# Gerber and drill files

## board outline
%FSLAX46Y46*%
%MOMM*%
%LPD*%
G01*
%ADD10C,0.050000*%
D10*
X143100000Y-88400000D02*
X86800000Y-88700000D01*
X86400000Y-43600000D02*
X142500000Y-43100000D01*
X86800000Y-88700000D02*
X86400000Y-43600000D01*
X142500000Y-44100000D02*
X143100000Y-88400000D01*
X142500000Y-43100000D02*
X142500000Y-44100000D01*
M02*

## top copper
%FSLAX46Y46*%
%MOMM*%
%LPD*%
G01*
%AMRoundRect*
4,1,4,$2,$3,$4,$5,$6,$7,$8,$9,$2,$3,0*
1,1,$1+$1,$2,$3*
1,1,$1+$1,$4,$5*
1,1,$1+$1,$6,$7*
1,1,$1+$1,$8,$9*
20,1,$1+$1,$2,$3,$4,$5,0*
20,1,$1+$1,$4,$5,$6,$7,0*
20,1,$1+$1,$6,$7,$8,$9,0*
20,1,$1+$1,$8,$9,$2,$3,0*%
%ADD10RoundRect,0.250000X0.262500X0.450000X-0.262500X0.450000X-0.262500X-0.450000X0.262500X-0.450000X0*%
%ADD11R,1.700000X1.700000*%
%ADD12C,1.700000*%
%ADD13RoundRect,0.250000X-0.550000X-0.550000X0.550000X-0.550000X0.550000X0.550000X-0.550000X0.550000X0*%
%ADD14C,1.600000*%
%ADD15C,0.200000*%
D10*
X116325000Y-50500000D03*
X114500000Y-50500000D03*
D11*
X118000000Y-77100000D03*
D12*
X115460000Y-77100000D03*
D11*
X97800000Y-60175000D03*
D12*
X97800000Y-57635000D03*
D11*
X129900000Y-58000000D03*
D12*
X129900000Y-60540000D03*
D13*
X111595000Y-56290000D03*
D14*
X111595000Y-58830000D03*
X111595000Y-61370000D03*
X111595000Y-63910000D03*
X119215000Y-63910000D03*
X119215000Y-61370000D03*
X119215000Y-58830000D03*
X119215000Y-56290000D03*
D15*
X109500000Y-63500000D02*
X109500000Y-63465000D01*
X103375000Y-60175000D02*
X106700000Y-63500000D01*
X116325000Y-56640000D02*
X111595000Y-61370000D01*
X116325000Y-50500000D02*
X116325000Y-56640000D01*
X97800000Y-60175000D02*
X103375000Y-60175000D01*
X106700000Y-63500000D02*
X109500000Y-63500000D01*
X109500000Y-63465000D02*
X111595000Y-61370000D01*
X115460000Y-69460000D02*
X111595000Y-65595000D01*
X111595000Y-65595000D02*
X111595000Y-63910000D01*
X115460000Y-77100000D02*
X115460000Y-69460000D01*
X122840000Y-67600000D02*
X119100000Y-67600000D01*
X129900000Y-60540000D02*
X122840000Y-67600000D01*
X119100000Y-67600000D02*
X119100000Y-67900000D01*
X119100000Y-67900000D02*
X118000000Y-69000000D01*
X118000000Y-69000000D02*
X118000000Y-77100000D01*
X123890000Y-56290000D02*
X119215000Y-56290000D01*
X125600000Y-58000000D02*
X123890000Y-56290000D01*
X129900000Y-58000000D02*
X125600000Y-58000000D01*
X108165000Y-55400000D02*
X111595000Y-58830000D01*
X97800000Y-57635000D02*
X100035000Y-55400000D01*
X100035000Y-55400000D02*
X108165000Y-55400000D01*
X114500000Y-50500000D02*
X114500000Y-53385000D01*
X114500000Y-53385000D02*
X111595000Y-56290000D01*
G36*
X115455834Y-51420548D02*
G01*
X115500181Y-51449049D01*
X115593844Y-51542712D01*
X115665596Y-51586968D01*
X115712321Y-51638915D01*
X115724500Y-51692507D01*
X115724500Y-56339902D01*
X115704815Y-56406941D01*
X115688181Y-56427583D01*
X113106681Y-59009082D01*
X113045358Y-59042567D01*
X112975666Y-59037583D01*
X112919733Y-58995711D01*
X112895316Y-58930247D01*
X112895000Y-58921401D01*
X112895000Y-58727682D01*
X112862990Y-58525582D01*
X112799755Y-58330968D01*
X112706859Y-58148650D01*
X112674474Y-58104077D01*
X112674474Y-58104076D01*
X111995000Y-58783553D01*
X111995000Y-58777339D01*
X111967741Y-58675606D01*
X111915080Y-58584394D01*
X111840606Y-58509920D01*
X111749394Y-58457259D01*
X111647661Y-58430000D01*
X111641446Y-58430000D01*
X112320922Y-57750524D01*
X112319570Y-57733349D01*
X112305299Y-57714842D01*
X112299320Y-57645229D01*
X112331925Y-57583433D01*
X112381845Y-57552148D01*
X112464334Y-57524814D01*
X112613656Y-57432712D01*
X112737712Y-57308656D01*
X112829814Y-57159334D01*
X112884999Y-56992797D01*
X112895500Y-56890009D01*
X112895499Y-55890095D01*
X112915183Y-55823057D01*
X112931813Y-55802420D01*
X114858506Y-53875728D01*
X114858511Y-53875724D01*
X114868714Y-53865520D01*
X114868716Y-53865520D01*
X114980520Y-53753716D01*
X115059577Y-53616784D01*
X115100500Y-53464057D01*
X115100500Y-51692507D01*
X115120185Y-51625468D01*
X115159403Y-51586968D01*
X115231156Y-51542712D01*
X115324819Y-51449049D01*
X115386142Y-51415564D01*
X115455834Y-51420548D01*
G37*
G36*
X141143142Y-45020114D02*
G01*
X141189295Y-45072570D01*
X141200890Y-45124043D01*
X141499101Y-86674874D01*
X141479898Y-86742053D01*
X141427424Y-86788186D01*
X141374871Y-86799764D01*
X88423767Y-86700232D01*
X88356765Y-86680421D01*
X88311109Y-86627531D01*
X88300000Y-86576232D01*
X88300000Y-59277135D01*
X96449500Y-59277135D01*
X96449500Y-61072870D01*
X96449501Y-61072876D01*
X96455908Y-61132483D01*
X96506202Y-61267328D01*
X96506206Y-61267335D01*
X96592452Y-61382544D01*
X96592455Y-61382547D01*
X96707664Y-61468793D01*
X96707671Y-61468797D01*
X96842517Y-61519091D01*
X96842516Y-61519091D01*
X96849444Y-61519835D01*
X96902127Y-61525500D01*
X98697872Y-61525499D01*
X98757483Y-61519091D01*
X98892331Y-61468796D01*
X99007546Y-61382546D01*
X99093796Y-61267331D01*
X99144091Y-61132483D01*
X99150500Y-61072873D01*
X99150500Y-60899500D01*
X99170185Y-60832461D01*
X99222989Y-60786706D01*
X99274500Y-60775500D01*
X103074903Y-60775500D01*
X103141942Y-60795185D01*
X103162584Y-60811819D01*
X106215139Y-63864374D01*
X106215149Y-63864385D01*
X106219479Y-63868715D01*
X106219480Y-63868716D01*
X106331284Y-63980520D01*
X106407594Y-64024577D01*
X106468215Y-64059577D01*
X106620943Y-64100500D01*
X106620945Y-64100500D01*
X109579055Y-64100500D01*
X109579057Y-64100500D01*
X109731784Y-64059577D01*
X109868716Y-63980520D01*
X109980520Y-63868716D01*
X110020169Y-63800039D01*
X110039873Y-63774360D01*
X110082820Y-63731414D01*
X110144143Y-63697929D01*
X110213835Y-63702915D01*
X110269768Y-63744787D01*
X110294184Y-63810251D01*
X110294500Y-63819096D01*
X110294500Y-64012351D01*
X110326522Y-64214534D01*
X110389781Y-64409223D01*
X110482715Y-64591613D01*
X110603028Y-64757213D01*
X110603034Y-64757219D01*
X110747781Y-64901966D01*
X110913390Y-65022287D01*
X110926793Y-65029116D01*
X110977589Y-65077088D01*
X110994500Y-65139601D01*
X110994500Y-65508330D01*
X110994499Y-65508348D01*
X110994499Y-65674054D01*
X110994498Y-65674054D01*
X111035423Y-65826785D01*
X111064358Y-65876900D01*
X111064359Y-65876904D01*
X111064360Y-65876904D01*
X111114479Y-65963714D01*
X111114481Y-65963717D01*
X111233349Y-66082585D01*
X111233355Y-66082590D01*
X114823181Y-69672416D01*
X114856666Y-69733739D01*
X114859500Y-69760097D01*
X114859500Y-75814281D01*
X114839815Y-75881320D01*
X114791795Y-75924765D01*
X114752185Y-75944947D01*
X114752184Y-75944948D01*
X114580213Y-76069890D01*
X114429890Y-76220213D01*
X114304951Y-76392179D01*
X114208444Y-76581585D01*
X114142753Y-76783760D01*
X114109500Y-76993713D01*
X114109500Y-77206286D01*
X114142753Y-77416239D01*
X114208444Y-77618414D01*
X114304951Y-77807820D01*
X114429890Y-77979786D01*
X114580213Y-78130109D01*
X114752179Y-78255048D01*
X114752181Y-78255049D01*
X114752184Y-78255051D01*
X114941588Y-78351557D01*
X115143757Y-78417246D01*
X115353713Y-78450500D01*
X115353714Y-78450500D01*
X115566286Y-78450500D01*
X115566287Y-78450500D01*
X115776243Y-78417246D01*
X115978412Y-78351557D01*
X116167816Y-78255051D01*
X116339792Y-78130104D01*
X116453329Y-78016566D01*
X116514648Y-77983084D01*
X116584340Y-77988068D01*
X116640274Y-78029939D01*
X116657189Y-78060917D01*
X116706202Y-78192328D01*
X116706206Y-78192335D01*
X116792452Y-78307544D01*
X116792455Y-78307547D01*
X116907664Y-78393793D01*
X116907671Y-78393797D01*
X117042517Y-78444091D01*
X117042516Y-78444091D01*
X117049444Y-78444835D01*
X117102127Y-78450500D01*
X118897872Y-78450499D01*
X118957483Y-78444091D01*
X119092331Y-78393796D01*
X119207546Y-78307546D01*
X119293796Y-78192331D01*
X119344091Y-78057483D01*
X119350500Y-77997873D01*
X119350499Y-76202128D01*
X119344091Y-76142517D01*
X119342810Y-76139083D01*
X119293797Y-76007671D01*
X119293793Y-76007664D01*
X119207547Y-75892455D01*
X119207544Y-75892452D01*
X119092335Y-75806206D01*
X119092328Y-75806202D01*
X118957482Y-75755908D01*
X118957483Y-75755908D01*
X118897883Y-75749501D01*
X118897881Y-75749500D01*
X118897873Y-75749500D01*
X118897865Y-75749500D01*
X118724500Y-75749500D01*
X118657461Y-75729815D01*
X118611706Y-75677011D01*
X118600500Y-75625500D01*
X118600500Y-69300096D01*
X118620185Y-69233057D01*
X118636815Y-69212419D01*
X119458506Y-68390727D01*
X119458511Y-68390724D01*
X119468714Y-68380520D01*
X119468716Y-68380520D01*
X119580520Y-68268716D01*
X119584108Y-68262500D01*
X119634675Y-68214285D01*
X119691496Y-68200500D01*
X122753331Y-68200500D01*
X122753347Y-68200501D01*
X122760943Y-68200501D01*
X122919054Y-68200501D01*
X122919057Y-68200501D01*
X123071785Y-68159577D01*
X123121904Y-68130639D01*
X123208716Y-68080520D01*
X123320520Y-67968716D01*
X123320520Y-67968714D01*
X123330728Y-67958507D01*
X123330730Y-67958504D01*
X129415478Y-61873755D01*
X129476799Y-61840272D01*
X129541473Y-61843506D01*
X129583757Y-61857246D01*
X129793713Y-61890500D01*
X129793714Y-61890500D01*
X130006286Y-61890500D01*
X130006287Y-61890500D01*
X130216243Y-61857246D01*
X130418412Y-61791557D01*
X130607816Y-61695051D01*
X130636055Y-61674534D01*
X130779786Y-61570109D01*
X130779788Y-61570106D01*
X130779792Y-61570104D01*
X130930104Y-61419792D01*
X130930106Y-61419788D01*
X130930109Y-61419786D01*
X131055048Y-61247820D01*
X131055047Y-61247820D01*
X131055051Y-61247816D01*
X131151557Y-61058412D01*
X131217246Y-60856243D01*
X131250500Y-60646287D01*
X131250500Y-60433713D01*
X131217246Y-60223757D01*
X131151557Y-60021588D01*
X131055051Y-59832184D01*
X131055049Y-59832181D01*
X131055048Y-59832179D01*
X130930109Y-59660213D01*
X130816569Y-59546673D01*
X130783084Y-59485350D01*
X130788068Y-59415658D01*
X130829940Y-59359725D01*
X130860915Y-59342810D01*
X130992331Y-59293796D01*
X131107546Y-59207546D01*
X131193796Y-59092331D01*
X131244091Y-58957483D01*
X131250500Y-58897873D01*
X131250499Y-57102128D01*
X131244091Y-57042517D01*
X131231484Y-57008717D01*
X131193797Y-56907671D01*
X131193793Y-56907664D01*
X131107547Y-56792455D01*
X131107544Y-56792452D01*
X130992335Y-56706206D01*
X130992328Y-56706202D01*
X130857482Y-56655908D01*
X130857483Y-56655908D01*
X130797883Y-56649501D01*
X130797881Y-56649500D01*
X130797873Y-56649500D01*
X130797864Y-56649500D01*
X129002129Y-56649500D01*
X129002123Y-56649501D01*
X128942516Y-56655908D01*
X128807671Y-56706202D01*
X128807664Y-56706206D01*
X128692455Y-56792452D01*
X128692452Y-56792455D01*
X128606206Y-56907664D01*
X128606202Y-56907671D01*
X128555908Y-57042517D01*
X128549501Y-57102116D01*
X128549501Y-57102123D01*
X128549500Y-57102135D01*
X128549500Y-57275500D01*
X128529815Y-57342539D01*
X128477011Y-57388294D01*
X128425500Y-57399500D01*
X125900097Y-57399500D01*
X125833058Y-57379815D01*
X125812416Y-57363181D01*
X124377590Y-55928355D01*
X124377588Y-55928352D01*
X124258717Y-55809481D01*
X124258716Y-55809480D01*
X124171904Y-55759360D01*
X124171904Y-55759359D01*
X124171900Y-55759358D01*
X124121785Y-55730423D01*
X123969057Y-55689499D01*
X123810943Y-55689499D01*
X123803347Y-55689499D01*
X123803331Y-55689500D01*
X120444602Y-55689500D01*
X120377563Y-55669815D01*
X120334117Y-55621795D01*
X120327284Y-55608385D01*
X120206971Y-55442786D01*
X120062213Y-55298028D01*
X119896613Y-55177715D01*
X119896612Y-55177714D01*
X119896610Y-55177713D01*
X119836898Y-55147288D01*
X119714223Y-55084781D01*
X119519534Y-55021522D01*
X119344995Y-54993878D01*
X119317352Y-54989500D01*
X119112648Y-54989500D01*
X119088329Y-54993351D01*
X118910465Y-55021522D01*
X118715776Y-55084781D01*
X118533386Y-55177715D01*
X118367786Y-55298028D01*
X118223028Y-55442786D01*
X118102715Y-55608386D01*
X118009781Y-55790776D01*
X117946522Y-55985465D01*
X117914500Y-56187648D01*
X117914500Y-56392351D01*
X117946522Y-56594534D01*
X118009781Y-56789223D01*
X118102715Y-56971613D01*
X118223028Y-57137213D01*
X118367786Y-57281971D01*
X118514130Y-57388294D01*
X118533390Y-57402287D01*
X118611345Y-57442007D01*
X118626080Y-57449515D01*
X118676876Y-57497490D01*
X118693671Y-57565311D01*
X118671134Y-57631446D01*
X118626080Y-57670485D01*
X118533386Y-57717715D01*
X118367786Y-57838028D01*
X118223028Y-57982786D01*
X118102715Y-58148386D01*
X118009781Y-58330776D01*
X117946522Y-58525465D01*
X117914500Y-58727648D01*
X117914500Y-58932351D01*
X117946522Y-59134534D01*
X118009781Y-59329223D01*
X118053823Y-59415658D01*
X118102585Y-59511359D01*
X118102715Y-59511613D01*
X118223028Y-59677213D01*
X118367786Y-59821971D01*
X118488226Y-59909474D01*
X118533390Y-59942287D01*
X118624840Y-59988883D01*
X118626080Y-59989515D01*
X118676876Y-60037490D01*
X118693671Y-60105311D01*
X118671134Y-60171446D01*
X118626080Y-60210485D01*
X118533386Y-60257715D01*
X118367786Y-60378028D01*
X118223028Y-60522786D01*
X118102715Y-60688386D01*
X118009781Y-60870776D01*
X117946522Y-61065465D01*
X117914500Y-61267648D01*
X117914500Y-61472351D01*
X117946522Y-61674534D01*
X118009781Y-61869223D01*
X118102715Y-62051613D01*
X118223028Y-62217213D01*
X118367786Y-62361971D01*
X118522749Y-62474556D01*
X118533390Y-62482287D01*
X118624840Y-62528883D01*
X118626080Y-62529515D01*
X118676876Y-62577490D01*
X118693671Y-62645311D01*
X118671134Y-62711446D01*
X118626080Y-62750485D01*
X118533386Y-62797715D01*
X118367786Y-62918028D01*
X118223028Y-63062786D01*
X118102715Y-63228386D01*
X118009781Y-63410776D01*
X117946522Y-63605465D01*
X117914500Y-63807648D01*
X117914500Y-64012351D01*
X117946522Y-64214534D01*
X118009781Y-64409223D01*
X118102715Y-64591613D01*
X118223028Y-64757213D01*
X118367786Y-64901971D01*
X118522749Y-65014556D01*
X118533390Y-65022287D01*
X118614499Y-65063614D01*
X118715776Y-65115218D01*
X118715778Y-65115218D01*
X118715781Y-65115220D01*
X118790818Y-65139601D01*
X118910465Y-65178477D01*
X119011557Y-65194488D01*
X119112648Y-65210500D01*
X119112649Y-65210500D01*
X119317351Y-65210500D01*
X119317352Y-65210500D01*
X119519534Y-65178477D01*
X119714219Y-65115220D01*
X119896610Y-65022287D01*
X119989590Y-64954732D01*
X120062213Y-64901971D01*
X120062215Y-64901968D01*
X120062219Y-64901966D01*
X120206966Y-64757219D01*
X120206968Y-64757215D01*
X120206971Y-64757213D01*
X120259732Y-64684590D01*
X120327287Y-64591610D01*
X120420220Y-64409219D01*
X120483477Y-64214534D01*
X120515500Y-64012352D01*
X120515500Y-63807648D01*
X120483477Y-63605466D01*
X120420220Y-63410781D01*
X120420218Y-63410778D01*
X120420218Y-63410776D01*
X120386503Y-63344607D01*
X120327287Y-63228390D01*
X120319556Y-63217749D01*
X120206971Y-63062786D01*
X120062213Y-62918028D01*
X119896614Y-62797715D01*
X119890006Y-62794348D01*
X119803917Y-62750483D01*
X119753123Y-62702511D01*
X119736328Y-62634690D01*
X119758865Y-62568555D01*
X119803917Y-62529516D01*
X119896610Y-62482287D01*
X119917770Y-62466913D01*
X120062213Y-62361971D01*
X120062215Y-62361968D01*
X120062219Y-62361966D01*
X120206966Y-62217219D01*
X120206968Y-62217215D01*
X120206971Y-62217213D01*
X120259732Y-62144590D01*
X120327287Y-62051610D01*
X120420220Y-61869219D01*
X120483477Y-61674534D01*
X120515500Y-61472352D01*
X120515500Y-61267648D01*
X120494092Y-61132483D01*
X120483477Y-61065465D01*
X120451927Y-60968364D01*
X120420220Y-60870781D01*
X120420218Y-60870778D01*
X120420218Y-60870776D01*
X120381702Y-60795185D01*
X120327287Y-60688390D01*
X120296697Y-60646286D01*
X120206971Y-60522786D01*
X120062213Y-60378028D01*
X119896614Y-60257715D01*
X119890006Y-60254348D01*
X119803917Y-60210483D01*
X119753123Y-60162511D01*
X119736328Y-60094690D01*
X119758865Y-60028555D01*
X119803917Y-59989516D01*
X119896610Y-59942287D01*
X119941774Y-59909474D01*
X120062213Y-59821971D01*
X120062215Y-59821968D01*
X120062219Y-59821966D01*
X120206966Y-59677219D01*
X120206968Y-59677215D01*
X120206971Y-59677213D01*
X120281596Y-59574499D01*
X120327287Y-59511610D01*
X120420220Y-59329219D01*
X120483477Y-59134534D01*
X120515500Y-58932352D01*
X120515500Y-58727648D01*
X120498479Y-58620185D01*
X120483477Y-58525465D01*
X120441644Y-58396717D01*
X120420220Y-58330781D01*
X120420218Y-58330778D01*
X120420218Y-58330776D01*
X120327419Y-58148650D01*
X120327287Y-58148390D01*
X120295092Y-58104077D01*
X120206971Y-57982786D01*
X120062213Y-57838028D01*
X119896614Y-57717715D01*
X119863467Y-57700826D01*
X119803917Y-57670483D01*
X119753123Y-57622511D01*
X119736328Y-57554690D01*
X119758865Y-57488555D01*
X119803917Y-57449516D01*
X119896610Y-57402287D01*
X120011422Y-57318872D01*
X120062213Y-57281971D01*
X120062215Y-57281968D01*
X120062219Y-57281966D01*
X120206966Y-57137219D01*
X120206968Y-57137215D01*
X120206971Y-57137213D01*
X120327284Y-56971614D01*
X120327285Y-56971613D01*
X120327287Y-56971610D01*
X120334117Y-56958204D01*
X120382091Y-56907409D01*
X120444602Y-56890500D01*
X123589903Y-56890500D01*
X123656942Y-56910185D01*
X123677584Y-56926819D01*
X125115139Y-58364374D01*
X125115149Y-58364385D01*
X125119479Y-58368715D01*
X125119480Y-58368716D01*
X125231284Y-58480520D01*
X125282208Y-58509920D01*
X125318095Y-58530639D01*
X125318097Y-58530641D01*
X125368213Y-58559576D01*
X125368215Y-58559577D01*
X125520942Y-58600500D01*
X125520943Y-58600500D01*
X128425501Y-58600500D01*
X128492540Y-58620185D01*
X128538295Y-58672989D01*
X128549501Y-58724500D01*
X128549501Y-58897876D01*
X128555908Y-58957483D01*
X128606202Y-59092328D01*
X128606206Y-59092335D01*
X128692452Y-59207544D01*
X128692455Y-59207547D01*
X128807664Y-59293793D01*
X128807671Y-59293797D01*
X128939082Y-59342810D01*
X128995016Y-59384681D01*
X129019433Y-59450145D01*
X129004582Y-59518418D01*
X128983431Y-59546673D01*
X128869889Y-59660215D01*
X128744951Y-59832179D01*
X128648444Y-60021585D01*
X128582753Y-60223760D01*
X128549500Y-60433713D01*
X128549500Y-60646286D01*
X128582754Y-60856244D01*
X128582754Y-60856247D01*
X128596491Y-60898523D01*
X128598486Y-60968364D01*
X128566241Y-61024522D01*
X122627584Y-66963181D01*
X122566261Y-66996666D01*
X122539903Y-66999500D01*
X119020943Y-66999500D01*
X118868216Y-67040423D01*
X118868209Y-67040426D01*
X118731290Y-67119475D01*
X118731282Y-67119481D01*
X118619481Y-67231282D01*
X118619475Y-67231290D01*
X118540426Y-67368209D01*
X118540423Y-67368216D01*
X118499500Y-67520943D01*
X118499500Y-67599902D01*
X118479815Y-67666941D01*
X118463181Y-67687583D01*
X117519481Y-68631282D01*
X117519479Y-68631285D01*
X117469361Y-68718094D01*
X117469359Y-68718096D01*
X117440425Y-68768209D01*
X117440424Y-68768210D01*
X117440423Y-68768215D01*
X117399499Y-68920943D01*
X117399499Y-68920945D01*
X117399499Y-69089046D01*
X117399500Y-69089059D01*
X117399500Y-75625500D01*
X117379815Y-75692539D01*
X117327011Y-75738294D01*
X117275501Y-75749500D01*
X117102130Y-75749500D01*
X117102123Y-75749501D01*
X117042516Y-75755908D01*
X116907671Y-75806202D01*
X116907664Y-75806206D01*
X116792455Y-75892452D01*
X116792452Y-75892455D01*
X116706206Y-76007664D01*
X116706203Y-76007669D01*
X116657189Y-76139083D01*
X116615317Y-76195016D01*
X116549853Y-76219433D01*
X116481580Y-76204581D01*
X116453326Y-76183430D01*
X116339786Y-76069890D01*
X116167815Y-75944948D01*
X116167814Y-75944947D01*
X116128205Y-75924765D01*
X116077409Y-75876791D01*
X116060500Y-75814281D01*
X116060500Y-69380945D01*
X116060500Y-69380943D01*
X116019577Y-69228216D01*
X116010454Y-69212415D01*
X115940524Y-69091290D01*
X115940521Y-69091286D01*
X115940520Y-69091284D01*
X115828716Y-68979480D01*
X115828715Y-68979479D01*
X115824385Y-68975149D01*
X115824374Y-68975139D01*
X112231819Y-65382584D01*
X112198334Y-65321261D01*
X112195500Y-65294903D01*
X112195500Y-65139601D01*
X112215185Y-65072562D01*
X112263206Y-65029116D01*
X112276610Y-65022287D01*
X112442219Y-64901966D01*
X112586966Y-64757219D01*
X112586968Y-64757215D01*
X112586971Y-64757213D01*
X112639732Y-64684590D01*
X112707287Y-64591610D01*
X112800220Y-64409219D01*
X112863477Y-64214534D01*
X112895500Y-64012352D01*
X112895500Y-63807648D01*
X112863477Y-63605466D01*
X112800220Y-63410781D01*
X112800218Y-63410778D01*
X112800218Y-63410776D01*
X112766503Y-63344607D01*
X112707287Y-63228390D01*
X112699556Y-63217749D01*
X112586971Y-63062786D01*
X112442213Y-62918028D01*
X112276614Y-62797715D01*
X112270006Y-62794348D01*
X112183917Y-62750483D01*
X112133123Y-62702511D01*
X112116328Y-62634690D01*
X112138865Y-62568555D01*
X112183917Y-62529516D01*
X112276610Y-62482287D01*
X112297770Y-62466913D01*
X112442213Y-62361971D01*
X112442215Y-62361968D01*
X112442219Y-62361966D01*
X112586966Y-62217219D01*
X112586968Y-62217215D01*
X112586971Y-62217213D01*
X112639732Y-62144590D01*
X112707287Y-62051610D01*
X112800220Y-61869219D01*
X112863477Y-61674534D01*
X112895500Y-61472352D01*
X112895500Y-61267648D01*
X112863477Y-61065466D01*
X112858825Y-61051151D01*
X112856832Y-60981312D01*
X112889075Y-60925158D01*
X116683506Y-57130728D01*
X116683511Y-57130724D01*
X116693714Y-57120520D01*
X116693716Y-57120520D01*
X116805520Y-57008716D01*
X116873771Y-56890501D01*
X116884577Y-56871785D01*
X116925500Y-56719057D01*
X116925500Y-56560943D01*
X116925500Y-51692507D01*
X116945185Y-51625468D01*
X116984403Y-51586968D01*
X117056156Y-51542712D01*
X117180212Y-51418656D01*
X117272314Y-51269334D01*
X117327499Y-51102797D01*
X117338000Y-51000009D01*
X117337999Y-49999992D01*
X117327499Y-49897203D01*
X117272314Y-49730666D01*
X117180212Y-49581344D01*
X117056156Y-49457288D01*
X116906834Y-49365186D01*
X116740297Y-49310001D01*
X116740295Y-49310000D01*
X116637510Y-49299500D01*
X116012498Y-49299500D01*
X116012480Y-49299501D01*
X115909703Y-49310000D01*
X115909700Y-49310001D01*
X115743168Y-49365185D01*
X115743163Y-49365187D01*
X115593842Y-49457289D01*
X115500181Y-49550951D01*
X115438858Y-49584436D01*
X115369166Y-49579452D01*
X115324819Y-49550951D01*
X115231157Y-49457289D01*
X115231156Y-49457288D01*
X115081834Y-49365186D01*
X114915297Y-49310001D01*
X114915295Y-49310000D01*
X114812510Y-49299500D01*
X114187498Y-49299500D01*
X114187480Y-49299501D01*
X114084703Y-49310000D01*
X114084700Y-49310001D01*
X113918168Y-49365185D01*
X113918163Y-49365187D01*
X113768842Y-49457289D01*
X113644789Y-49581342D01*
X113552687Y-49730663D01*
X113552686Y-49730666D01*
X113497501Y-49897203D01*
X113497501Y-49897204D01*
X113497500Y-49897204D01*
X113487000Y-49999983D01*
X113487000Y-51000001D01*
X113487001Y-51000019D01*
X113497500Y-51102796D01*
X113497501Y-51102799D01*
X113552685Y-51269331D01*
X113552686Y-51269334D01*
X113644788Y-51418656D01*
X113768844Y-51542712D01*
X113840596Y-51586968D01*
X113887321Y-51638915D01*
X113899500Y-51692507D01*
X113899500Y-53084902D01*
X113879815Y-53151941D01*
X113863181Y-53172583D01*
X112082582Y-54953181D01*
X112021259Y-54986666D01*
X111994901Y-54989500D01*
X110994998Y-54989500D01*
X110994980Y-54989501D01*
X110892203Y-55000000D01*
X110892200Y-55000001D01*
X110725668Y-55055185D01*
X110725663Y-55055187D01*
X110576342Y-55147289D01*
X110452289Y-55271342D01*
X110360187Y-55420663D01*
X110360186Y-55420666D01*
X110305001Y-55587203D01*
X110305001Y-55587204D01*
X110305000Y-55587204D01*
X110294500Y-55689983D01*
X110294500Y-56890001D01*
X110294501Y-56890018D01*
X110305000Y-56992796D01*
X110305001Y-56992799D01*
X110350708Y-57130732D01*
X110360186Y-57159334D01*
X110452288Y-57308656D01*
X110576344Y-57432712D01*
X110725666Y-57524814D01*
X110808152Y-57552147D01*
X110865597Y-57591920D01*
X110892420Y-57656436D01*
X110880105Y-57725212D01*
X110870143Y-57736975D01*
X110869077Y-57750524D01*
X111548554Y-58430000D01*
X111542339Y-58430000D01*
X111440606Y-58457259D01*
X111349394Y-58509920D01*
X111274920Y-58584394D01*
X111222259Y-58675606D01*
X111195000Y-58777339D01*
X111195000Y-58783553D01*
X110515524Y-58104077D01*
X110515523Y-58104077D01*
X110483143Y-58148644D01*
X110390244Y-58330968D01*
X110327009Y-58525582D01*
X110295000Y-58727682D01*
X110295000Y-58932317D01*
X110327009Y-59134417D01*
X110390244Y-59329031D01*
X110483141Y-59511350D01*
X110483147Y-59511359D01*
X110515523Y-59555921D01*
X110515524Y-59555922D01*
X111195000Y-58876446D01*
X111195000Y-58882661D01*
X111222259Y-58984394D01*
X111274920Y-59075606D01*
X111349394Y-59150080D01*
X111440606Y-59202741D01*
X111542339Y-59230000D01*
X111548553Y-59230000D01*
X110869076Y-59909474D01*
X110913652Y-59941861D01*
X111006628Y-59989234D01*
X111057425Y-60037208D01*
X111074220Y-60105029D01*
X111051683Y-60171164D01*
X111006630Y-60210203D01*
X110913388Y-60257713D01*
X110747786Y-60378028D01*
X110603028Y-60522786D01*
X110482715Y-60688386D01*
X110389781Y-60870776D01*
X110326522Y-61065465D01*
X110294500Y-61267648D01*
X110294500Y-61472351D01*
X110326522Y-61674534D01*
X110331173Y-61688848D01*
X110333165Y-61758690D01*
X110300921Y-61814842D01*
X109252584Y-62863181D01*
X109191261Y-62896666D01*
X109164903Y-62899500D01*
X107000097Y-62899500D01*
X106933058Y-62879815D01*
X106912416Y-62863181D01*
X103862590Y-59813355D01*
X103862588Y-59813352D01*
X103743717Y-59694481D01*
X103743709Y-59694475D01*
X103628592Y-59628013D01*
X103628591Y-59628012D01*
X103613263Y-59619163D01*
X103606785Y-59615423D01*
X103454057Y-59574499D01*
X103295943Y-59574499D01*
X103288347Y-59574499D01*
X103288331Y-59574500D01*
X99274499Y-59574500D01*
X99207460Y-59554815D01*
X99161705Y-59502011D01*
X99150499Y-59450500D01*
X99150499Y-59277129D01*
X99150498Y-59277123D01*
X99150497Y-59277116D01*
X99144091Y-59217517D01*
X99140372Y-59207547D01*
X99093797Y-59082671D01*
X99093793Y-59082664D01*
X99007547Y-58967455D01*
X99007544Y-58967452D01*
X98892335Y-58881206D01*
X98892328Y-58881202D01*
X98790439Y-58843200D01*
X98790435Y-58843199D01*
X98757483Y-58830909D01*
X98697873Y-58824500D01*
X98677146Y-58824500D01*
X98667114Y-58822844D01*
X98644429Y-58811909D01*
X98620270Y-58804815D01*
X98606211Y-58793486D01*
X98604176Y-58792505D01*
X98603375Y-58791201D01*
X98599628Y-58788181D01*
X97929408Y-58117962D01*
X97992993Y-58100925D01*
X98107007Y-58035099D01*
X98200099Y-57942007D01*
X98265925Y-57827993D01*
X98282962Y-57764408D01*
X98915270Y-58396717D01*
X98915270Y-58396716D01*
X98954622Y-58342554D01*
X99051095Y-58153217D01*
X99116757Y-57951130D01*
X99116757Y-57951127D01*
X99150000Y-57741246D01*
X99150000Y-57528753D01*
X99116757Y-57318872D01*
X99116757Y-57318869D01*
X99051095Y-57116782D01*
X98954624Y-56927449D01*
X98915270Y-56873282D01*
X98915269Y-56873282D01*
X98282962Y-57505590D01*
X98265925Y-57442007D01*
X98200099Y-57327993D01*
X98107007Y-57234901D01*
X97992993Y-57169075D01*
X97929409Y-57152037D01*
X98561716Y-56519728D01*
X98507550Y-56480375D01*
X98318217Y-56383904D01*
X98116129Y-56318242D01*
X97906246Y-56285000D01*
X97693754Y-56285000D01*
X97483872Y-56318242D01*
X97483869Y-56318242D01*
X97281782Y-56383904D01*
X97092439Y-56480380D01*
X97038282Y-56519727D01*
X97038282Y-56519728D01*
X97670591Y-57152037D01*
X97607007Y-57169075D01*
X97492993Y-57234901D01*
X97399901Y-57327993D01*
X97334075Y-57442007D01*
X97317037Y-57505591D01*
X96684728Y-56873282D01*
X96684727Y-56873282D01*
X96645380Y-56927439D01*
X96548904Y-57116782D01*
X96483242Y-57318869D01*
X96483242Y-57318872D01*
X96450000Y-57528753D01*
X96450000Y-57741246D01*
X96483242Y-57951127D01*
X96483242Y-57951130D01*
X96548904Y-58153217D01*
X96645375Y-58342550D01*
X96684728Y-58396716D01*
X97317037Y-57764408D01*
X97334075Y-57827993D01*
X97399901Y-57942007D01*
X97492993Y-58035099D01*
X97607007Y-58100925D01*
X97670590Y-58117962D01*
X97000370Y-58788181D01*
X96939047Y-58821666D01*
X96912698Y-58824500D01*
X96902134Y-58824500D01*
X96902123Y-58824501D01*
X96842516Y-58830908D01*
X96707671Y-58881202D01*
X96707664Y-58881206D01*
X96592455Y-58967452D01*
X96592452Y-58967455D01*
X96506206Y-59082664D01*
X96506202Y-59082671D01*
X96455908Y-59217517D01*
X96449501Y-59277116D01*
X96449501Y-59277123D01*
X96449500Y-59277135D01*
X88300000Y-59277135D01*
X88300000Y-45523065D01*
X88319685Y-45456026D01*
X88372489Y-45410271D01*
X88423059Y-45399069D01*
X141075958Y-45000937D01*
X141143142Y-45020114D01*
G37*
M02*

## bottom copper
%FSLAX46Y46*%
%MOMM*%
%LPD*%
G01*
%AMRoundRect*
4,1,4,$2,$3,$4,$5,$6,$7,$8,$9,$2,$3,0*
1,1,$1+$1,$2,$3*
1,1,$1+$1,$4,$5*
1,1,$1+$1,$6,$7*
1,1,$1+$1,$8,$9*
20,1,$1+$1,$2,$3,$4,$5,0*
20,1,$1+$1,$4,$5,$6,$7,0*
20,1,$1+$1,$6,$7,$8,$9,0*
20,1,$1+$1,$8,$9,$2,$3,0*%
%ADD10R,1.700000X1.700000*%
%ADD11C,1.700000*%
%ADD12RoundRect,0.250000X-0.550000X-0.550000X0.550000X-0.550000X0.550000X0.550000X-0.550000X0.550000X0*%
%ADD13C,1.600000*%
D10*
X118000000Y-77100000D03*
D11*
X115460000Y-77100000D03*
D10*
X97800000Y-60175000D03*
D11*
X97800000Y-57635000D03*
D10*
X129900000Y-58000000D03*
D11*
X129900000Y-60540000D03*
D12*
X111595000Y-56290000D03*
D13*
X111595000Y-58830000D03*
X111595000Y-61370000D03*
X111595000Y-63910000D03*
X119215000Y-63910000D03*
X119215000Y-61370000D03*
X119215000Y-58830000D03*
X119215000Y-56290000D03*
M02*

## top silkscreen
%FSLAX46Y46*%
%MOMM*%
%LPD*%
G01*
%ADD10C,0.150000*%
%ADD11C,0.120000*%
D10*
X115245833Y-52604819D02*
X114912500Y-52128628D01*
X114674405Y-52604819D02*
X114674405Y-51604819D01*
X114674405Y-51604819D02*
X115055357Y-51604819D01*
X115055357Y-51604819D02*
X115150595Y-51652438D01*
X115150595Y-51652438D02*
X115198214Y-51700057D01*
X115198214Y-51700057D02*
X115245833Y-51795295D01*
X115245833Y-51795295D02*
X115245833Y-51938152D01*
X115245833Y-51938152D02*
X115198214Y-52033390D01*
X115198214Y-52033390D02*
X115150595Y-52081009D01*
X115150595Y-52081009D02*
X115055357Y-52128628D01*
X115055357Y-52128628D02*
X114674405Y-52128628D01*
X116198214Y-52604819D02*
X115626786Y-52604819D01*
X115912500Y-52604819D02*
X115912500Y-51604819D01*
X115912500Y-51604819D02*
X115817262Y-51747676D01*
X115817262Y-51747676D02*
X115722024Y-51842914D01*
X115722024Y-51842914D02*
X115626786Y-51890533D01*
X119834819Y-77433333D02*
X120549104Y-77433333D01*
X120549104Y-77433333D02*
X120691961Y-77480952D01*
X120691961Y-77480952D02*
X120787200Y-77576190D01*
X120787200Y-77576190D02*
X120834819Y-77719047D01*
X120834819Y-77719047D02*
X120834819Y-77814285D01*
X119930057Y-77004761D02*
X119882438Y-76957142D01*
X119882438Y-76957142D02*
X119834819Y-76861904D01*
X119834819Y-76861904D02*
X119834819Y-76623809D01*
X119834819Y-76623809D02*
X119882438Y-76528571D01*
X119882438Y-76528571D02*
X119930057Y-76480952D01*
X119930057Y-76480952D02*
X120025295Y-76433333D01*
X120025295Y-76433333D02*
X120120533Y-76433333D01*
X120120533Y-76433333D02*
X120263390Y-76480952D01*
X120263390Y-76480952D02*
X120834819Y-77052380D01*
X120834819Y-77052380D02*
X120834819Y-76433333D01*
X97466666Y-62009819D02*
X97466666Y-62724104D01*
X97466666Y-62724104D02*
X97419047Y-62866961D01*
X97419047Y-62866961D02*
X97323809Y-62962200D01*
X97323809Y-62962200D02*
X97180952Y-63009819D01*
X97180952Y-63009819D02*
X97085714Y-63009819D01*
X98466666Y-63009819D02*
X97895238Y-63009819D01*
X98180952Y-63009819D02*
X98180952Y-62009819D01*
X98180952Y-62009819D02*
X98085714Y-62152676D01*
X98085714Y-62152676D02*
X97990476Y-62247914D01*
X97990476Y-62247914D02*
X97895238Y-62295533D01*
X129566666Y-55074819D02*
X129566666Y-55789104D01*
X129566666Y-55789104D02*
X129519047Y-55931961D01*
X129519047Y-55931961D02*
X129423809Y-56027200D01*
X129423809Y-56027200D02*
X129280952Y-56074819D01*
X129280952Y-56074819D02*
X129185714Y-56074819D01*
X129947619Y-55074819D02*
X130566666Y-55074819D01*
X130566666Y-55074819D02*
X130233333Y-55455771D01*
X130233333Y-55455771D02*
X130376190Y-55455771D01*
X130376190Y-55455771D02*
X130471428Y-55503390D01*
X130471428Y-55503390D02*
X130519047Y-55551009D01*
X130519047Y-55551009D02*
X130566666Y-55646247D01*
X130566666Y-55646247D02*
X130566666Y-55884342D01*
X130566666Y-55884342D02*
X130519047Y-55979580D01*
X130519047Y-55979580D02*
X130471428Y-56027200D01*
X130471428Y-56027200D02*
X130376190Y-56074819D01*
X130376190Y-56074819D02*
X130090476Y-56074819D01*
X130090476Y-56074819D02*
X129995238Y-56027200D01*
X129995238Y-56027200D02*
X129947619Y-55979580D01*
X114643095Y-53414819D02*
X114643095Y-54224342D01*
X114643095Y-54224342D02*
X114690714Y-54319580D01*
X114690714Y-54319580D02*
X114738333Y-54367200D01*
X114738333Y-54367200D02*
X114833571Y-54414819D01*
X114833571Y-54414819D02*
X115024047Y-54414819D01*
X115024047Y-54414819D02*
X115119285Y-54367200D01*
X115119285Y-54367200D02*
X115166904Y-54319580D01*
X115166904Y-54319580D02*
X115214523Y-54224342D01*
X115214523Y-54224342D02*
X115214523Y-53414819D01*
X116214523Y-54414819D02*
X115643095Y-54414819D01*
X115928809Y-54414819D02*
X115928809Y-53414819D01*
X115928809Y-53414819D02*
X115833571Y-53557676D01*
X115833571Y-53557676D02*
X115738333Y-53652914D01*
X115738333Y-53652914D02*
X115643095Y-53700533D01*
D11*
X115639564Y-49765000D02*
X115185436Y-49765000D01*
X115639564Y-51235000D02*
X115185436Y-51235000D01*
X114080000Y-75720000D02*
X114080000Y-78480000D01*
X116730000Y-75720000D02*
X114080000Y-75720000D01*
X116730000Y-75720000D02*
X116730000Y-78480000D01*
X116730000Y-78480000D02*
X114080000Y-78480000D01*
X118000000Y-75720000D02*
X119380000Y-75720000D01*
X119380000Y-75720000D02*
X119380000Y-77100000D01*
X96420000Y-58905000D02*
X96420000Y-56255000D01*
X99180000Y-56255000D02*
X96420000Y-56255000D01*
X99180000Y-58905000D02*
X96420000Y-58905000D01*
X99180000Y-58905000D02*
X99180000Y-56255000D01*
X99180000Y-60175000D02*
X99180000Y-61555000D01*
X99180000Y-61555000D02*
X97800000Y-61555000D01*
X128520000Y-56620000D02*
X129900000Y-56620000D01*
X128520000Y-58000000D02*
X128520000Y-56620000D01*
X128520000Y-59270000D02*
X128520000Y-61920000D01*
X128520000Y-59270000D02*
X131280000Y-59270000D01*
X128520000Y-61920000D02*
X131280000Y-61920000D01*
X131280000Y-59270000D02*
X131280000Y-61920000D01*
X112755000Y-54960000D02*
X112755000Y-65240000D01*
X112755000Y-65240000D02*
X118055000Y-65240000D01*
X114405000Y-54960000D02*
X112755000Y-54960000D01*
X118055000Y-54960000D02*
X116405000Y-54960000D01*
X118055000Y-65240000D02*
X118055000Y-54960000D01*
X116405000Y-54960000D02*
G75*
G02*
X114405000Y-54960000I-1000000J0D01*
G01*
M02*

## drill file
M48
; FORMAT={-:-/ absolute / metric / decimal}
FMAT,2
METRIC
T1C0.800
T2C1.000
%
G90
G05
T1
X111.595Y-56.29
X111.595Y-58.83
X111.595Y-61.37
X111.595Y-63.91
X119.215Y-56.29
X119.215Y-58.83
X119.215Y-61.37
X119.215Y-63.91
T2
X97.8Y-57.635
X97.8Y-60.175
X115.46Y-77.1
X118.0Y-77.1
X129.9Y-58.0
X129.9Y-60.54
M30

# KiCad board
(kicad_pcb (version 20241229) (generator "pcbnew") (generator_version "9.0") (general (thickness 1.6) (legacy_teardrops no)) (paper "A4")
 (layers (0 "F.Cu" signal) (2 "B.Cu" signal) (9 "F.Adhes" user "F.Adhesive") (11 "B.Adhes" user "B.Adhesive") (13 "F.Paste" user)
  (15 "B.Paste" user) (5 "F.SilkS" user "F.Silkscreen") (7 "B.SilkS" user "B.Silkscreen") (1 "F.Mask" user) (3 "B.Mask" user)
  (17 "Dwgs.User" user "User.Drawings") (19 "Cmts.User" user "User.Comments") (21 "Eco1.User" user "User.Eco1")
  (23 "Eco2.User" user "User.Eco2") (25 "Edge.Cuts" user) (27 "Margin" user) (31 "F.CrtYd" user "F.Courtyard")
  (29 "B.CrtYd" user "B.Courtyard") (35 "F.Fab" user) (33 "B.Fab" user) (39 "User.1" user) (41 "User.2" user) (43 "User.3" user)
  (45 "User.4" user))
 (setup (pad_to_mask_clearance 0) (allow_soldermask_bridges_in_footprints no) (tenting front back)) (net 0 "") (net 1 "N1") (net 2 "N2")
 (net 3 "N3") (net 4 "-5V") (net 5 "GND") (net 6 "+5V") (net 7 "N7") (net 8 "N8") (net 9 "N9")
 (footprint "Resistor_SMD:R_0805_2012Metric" (layer "F.Cu") (at 115.4125 50.5 180)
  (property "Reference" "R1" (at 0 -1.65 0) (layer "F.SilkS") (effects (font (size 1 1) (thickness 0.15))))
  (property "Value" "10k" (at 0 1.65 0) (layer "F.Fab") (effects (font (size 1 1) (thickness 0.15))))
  (fp_line (start -0.227064 0.735) (end 0.227064 0.735) (stroke (width 0.12) (type solid)) (layer "F.SilkS"))
  (fp_line (start -0.227064 -0.735) (end 0.227064 -0.735) (stroke (width 0.12) (type solid)) (layer "F.SilkS"))
  (pad "1" smd roundrect (at -0.9125 0 180) (size 1.025 1.4) (layers "F.Cu" "F.Mask" "F.Paste") (roundrect_rratio 0.243902) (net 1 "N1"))
  (pad "2" smd roundrect (at 0.9125 0 180) (size 1.025 1.4) (layers "F.Cu" "F.Mask" "F.Paste") (roundrect_rratio 0.243902) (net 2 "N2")))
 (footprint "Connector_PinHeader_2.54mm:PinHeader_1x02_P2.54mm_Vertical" (layer "F.Cu") (at 118 77.1 -90)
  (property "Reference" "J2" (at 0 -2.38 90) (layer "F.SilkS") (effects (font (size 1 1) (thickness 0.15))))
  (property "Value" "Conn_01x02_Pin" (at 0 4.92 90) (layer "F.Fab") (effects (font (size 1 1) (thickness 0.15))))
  (fp_line (start -1.38 3.92) (end 1.38 3.92) (stroke (width 0.12) (type solid)) (layer "F.SilkS"))
  (fp_line (start -1.38 1.27) (end -1.38 3.92) (stroke (width 0.12) (type solid)) (layer "F.SilkS"))
  (fp_line (start -1.38 1.27) (end 1.38 1.27) (stroke (width 0.12) (type solid)) (layer "F.SilkS"))
  (fp_line (start 1.38 1.27) (end 1.38 3.92) (stroke (width 0.12) (type solid)) (layer "F.SilkS"))
  (fp_line (start -1.38 0) (end -1.38 -1.38) (stroke (width 0.12) (type solid)) (layer "F.SilkS"))
  (fp_line (start -1.38 -1.38) (end 0 -1.38) (stroke (width 0.12) (type solid)) (layer "F.SilkS"))
  (pad "1" thru_hole rect (at 0 0 270) (size 1.7 1.7) (drill 1) (layers "*.Cu" "*.Mask") (remove_unused_layers no) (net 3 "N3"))
  (pad "2" thru_hole circle (at 0 2.54 270) (size 1.7 1.7) (drill 1) (layers "*.Cu" "*.Mask") (remove_unused_layers no) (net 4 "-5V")))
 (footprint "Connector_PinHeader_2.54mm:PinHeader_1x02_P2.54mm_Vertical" (layer "F.Cu") (at 97.8 60.175 180)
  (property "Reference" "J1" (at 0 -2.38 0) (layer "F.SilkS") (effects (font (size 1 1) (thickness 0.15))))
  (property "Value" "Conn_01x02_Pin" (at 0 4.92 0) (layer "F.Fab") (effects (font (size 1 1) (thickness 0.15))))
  (fp_line (start 1.38 1.27) (end 1.38 3.92) (stroke (width 0.12) (type solid)) (layer "F.SilkS"))
  (fp_line (start -1.38 3.92) (end 1.38 3.92) (stroke (width 0.12) (type solid)) (layer "F.SilkS"))
  (fp_line (start -1.38 1.27) (end 1.38 1.27) (stroke (width 0.12) (type solid)) (layer "F.SilkS"))
  (fp_line (start -1.38 1.27) (end -1.38 3.92) (stroke (width 0.12) (type solid)) (layer "F.SilkS"))
  (fp_line (start -1.38 0) (end -1.38 -1.38) (stroke (width 0.12) (type solid)) (layer "F.SilkS"))
  (fp_line (start -1.38 -1.38) (end 0 -1.38) (stroke (width 0.12) (type solid)) (layer "F.SilkS"))
  (pad "1" thru_hole rect (at 0 0 180) (size 1.7 1.7) (drill 1) (layers "*.Cu" "*.Mask") (remove_unused_layers no) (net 1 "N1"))
  (pad "2" thru_hole circle (at 0 2.54 180) (size 1.7 1.7) (drill 1) (layers "*.Cu" "*.Mask") (remove_unused_layers no) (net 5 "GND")))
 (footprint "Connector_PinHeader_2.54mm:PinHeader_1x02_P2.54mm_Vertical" (layer "F.Cu") (at 129.9 58)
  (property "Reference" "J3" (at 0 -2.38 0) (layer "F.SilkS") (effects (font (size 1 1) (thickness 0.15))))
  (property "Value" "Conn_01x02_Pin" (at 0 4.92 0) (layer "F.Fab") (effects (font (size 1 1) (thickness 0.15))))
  (fp_line (start -1.38 -1.38) (end 0 -1.38) (stroke (width 0.12) (type solid)) (layer "F.SilkS"))
  (fp_line (start -1.38 0) (end -1.38 -1.38) (stroke (width 0.12) (type solid)) (layer "F.SilkS"))
  (fp_line (start -1.38 1.27) (end -1.38 3.92) (stroke (width 0.12) (type solid)) (layer "F.SilkS"))
  (fp_line (start -1.38 1.27) (end 1.38 1.27) (stroke (width 0.12) (type solid)) (layer "F.SilkS"))
  (fp_line (start -1.38 3.92) (end 1.38 3.92) (stroke (width 0.12) (type solid)) (layer "F.SilkS"))
  (fp_line (start 1.38 1.27) (end 1.38 3.92) (stroke (width 0.12) (type solid)) (layer "F.SilkS"))
  (pad "1" thru_hole rect (at 0 0) (size 1.7 1.7) (drill 1) (layers "*.Cu" "*.Mask") (remove_unused_layers no) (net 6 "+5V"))
  (pad "2" thru_hole circle (at 0 2.54) (size 1.7 1.7) (drill 1) (layers "*.Cu" "*.Mask") (remove_unused_layers no) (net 3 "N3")))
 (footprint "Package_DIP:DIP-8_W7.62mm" (layer "F.Cu") (at 111.595 56.29)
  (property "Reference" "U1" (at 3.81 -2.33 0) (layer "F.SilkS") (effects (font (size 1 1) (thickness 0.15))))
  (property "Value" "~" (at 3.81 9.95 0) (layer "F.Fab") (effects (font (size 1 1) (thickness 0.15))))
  (fp_line (start 1.16 -1.33) (end 1.16 8.95) (stroke (width 0.12) (type solid)) (layer "F.SilkS"))
  (fp_line (start 1.16 8.95) (end 6.46 8.95) (stroke (width 0.12) (type solid)) (layer "F.SilkS"))
  (fp_line (start 2.81 -1.33) (end 1.16 -1.33) (stroke (width 0.12) (type solid)) (layer "F.SilkS"))
  (fp_line (start 6.46 -1.33) (end 4.81 -1.33) (stroke (width 0.12) (type solid)) (layer "F.SilkS"))
  (fp_line (start 6.46 8.95) (end 6.46 -1.33) (stroke (width 0.12) (type solid)) (layer "F.SilkS"))
  (fp_arc (start 4.81 -1.33) (mid 3.81 -0.33) (end 2.81 -1.33) (stroke (width 0.12) (type solid)) (layer "F.SilkS"))
  (pad "1" thru_hole roundrect (at 0 0) (size 1.6 1.6) (drill 0.8) (layers "*.Cu" "*.Mask") (remove_unused_layers no)
   (roundrect_rratio 0.15625) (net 2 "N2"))
  (pad "2" thru_hole circle (at 0 2.54) (size 1.6 1.6) (drill 0.8) (layers "*.Cu" "*.Mask") (remove_unused_layers no) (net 5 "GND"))
  (pad "3" thru_hole circle (at 0 5.08) (size 1.6 1.6) (drill 0.8) (layers "*.Cu" "*.Mask") (remove_unused_layers no) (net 1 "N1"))
  (pad "4" thru_hole circle (at 0 7.62) (size 1.6 1.6) (drill 0.8) (layers "*.Cu" "*.Mask") (remove_unused_layers no) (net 4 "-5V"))
  (pad "5" thru_hole circle (at 7.62 7.62) (size 1.6 1.6) (drill 0.8) (layers "*.Cu" "*.Mask") (remove_unused_layers no) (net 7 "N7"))
  (pad "6" thru_hole circle (at 7.62 5.08) (size 1.6 1.6) (drill 0.8) (layers "*.Cu" "*.Mask") (remove_unused_layers no) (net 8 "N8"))
  (pad "7" thru_hole circle (at 7.62 2.54) (size 1.6 1.6) (drill 0.8) (layers "*.Cu" "*.Mask") (remove_unused_layers no) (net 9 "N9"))
  (pad "8" thru_hole circle (at 7.62 0) (size 1.6 1.6) (drill 0.8) (layers "*.Cu" "*.Mask") (remove_unused_layers no) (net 6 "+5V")))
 (gr_line (start 143.1 88.4) (end 86.8 88.7) (stroke (width 0.05) (type default)) (layer "Edge.Cuts"))
 (gr_line (start 86.4 43.6) (end 142.5 43.1) (stroke (width 0.05) (type default)) (layer "Edge.Cuts"))
 (gr_line (start 86.8 88.7) (end 86.4 43.6) (stroke (width 0.05) (type default)) (layer "Edge.Cuts"))
 (gr_line (start 142.5 44.1) (end 143.1 88.4) (stroke (width 0.05) (type default)) (layer "Edge.Cuts"))
 (gr_line (start 142.5 43.1) (end 142.5 44.1) (stroke (width 0.05) (type default)) (layer "Edge.Cuts"))
 (segment (start 109.5 63.5) (end 109.5 63.465) (width 0.2) (layer "F.Cu") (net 1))
 (segment (start 103.375 60.175) (end 106.7 63.5) (width 0.2) (layer "F.Cu") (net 1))
 (segment (start 116.325 56.64) (end 111.595 61.37) (width 0.2) (layer "F.Cu") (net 1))
 (segment (start 116.325 50.5) (end 116.325 56.64) (width 0.2) (layer "F.Cu") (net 1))
 (segment (start 97.8 60.175) (end 103.375 60.175) (width 0.2) (layer "F.Cu") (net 1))
 (segment (start 106.7 63.5) (end 109.5 63.5) (width 0.2) (layer "F.Cu") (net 1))
 (segment (start 109.5 63.465) (end 111.595 61.37) (width 0.2) (layer "F.Cu") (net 1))
 (segment (start 115.46 69.46) (end 111.595 65.595) (width 0.2) (layer "F.Cu") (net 4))
 (segment (start 111.595 65.595) (end 111.595 63.91) (width 0.2) (layer "F.Cu") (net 4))
 (segment (start 115.46 77.1) (end 115.46 69.46) (width 0.2) (layer "F.Cu") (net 4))
 (segment (start 122.84 67.6) (end 119.1 67.6) (width 0.2) (layer "F.Cu") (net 3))
 (segment (start 129.9 60.54) (end 122.84 67.6) (width 0.2) (layer "F.Cu") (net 3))
 (segment (start 119.1 67.6) (end 119.1 67.9) (width 0.2) (layer "F.Cu") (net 3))
 (segment (start 119.1 67.9) (end 118 69) (width 0.2) (layer "F.Cu") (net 3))
 (segment (start 118 69) (end 118 77.1) (width 0.2) (layer "F.Cu") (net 3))
 (segment (start 123.89 56.29) (end 119.215 56.29) (width 0.2) (layer "F.Cu") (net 6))
 (segment (start 125.6 58) (end 123.89 56.29) (width 0.2) (layer "F.Cu") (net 6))
 (segment (start 129.9 58) (end 125.6 58) (width 0.2) (layer "F.Cu") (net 6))
 (segment (start 108.165 55.4) (end 111.595 58.83) (width 0.2) (layer "F.Cu") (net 5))
 (segment (start 97.8 57.635) (end 100.035 55.4) (width 0.2) (layer "F.Cu") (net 5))
 (segment (start 100.035 55.4) (end 108.165 55.4) (width 0.2) (layer "F.Cu") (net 5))
 (segment (start 114.5 50.5) (end 114.5 53.385) (width 0.2) (layer "F.Cu") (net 2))
 (segment (start 114.5 53.385) (end 111.595 56.29) (width 0.2) (layer "F.Cu") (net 2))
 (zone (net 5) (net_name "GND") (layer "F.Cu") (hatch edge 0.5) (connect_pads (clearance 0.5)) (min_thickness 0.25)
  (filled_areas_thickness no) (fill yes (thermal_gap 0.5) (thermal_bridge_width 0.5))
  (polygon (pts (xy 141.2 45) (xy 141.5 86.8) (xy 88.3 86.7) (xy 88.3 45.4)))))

